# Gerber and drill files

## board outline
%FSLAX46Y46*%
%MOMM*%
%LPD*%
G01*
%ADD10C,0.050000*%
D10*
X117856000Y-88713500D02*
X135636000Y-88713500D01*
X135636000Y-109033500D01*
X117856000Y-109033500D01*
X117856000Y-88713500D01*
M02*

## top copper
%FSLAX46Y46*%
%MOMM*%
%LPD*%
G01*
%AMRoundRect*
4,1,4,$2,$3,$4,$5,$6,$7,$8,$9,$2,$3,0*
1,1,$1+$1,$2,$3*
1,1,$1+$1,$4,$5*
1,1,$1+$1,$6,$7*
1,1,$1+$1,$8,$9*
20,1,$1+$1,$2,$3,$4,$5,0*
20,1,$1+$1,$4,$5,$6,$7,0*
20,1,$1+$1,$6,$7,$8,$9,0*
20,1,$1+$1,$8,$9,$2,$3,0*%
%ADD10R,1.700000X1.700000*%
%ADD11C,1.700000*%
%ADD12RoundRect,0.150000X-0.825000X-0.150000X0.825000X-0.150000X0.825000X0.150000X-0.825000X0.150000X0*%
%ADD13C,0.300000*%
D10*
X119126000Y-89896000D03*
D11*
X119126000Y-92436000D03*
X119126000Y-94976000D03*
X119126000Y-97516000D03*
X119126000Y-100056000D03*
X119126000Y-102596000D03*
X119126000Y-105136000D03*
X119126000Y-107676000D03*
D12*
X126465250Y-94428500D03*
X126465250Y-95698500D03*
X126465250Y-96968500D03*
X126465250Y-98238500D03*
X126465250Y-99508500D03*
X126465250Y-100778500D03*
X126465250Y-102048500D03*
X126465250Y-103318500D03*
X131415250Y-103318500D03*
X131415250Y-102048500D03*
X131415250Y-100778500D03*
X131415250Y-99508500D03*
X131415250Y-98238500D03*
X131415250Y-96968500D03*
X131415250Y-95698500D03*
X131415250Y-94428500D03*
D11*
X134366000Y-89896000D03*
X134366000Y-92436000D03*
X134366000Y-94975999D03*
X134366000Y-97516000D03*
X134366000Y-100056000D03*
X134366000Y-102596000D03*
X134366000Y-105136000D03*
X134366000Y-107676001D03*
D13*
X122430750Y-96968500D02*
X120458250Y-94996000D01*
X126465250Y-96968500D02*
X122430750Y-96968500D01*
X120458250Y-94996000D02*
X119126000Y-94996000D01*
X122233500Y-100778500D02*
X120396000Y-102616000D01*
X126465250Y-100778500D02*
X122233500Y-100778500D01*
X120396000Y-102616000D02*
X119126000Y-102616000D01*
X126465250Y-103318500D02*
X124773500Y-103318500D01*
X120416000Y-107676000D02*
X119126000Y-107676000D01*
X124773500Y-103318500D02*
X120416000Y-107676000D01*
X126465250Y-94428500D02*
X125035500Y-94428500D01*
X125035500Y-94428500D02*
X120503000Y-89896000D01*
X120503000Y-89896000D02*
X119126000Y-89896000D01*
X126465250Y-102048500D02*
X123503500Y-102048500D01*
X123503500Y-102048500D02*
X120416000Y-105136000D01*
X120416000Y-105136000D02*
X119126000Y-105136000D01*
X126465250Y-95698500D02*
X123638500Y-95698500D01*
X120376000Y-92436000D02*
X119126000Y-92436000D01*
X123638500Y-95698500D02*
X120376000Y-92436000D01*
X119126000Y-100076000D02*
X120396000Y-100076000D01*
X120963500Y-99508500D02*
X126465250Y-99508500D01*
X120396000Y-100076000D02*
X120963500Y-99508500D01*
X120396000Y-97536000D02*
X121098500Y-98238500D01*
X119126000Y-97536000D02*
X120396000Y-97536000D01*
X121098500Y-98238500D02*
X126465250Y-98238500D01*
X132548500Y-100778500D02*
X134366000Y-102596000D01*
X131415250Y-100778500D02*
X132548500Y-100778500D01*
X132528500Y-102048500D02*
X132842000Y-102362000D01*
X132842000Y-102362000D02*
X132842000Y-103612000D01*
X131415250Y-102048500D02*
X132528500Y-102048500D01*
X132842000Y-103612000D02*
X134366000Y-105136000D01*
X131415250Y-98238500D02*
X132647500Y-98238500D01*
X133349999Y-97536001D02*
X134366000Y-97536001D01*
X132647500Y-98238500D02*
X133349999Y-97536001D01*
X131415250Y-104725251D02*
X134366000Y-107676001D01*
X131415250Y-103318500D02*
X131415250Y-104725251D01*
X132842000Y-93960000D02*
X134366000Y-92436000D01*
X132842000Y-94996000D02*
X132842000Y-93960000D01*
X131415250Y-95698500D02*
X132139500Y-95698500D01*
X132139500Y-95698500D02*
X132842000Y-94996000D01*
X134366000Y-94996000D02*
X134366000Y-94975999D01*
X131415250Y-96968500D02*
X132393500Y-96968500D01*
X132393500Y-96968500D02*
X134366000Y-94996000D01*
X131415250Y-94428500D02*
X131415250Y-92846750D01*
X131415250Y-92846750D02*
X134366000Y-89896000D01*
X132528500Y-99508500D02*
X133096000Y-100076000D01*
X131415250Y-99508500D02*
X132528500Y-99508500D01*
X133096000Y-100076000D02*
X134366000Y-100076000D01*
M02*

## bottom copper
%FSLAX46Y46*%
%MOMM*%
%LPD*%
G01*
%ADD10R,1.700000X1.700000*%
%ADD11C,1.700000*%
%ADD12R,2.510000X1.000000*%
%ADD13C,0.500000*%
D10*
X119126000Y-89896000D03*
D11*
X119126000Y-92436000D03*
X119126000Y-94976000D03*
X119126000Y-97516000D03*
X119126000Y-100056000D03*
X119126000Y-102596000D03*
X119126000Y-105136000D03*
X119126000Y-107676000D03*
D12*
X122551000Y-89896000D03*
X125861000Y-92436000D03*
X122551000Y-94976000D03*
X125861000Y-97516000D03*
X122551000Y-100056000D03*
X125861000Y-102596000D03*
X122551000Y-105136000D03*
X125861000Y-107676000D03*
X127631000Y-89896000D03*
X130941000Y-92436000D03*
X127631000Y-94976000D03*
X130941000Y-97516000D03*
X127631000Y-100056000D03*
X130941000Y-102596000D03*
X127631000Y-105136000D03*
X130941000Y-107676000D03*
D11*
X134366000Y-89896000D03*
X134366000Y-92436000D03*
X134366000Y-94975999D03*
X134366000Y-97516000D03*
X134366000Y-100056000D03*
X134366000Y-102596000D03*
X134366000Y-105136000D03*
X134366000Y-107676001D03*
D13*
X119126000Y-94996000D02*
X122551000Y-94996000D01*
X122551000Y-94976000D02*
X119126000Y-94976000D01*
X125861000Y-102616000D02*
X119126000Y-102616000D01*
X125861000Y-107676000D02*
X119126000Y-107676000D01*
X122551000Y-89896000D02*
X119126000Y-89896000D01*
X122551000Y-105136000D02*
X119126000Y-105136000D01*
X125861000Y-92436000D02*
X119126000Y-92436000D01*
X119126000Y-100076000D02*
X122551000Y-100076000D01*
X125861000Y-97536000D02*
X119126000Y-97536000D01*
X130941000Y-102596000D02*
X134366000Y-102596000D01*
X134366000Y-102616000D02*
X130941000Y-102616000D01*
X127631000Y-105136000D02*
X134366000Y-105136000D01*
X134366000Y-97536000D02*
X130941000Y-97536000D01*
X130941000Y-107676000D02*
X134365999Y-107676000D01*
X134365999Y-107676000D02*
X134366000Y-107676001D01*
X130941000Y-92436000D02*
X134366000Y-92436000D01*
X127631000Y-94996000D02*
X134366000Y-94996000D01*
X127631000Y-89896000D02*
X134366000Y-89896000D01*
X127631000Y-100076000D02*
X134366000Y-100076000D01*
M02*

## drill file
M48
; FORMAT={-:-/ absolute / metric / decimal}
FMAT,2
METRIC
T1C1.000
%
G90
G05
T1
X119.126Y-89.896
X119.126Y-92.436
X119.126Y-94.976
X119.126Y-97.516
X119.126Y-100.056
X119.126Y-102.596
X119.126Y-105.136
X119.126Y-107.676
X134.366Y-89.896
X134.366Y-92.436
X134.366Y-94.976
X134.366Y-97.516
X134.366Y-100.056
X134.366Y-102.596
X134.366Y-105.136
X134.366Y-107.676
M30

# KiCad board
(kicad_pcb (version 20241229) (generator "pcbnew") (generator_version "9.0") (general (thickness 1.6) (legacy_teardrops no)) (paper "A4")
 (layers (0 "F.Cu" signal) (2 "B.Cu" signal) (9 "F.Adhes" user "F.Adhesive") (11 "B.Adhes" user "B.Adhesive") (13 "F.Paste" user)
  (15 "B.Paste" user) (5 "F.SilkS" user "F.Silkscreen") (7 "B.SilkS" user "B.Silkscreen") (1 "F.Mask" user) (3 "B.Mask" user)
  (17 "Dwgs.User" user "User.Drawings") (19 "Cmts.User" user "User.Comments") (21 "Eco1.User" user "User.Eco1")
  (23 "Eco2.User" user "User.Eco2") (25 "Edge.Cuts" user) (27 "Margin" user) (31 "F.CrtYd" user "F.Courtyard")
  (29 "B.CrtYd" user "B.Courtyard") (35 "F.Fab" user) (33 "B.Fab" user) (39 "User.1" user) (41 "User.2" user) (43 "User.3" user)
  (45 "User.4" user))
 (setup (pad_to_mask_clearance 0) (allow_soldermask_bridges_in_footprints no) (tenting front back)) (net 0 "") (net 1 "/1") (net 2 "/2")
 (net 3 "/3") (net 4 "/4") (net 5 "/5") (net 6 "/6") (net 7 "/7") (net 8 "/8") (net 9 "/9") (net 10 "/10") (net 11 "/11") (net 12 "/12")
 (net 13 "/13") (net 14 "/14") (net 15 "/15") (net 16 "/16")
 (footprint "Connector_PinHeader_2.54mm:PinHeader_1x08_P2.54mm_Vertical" (layer "F.Cu") (at 119.126 89.896)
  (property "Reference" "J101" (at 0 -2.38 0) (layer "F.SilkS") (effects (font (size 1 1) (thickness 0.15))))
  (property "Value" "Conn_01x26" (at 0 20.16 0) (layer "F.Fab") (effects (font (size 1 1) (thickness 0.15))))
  (pad "1" thru_hole rect (at 0 0) (size 1.7 1.7) (drill 1) (layers "*.Cu" "*.Mask") (remove_unused_layers no) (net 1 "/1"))
  (pad "2" thru_hole circle (at 0 2.54) (size 1.7 1.7) (drill 1) (layers "*.Cu" "*.Mask") (remove_unused_layers no) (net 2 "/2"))
  (pad "3" thru_hole circle (at 0 5.08) (size 1.7 1.7) (drill 1) (layers "*.Cu" "*.Mask") (remove_unused_layers no) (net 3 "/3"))
  (pad "4" thru_hole circle (at 0 7.62) (size 1.7 1.7) (drill 1) (layers "*.Cu" "*.Mask") (remove_unused_layers no) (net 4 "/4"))
  (pad "5" thru_hole circle (at 0 10.16) (size 1.7 1.7) (drill 1) (layers "*.Cu" "*.Mask") (remove_unused_layers no) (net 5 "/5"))
  (pad "6" thru_hole circle (at 0 12.7) (size 1.7 1.7) (drill 1) (layers "*.Cu" "*.Mask") (remove_unused_layers no) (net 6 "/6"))
  (pad "7" thru_hole circle (at 0 15.24) (size 1.7 1.7) (drill 1) (layers "*.Cu" "*.Mask") (remove_unused_layers no) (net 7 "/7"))
  (pad "8" thru_hole circle (at 0 17.78) (size 1.7 1.7) (drill 1) (layers "*.Cu" "*.Mask") (remove_unused_layers no) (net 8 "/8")))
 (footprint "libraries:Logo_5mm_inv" (layer "F.Cu") (at 128.940483 91.168125)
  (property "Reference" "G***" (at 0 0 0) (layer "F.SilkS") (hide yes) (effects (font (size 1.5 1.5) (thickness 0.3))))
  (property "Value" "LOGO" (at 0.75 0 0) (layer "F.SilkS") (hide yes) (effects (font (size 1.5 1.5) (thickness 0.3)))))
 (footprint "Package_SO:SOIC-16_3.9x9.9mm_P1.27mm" (layer "F.Cu") (at 128.94025 98.8735)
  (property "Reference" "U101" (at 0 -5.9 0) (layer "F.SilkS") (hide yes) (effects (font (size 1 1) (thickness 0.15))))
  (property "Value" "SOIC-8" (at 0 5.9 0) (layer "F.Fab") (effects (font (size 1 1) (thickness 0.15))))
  (pad "1" smd roundrect (at -2.475 -4.445) (size 1.95 0.6) (layers "F.Cu" "F.Mask" "F.Paste") (roundrect_rratio 0.25) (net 1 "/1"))
  (pad "2" smd roundrect (at -2.475 -3.175) (size 1.95 0.6) (layers "F.Cu" "F.Mask" "F.Paste") (roundrect_rratio 0.25) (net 2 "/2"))
  (pad "3" smd roundrect (at -2.475 -1.905) (size 1.95 0.6) (layers "F.Cu" "F.Mask" "F.Paste") (roundrect_rratio 0.25) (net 3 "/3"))
  (pad "4" smd roundrect (at -2.475 -0.635) (size 1.95 0.6) (layers "F.Cu" "F.Mask" "F.Paste") (roundrect_rratio 0.25) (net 4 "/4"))
  (pad "5" smd roundrect (at -2.475 0.635) (size 1.95 0.6) (layers "F.Cu" "F.Mask" "F.Paste") (roundrect_rratio 0.25) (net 5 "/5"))
  (pad "6" smd roundrect (at -2.475 1.905) (size 1.95 0.6) (layers "F.Cu" "F.Mask" "F.Paste") (roundrect_rratio 0.25) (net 6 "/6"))
  (pad "7" smd roundrect (at -2.475 3.175) (size 1.95 0.6) (layers "F.Cu" "F.Mask" "F.Paste") (roundrect_rratio 0.25) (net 7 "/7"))
  (pad "8" smd roundrect (at -2.475 4.445) (size 1.95 0.6) (layers "F.Cu" "F.Mask" "F.Paste") (roundrect_rratio 0.25) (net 8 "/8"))
  (pad "9" smd roundrect (at 2.475 4.445) (size 1.95 0.6) (layers "F.Cu" "F.Mask" "F.Paste") (roundrect_rratio 0.25) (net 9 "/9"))
  (pad "10" smd roundrect (at 2.475 3.175) (size 1.95 0.6) (layers "F.Cu" "F.Mask" "F.Paste") (roundrect_rratio 0.25) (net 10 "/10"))
  (pad "11" smd roundrect (at 2.475 1.905) (size 1.95 0.6) (layers "F.Cu" "F.Mask" "F.Paste") (roundrect_rratio 0.25) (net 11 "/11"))
  (pad "12" smd roundrect (at 2.475 0.635) (size 1.95 0.6) (layers "F.Cu" "F.Mask" "F.Paste") (roundrect_rratio 0.25) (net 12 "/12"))
  (pad "13" smd roundrect (at 2.475 -0.635) (size 1.95 0.6) (layers "F.Cu" "F.Mask" "F.Paste") (roundrect_rratio 0.25) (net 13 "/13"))
  (pad "14" smd roundrect (at 2.475 -1.905) (size 1.95 0.6) (layers "F.Cu" "F.Mask" "F.Paste") (roundrect_rratio 0.25) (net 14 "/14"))
  (pad "15" smd roundrect (at 2.475 -3.175) (size 1.95 0.6) (layers "F.Cu" "F.Mask" "F.Paste") (roundrect_rratio 0.25) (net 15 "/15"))
  (pad "16" smd roundrect (at 2.475 -4.445) (size 1.95 0.6) (layers "F.Cu" "F.Mask" "F.Paste") (roundrect_rratio 0.25) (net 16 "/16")))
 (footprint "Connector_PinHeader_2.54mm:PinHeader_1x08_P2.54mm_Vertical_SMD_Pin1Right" (layer "B.Cu") (at 124.206 98.786 180)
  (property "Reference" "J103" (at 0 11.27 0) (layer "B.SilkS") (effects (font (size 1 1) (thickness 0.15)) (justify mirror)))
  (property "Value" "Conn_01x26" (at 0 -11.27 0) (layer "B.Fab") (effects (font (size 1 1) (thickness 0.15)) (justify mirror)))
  (pad "1" smd rect (at 1.655 8.89 180) (size 2.51 1) (layers "B.Cu" "B.Mask" "B.Paste") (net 1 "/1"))
  (pad "2" smd rect (at -1.655 6.35 180) (size 2.51 1) (layers "B.Cu" "B.Mask" "B.Paste") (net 2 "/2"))
  (pad "3" smd rect (at 1.655 3.81 180) (size 2.51 1) (layers "B.Cu" "B.Mask" "B.Paste") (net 3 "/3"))
  (pad "4" smd rect (at -1.655 1.27 180) (size 2.51 1) (layers "B.Cu" "B.Mask" "B.Paste") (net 4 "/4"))
  (pad "5" smd rect (at 1.655 -1.27 180) (size 2.51 1) (layers "B.Cu" "B.Mask" "B.Paste") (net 5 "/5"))
  (pad "6" smd rect (at -1.655 -3.81 180) (size 2.51 1) (layers "B.Cu" "B.Mask" "B.Paste") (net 6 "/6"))
  (pad "7" smd rect (at 1.655 -6.35 180) (size 2.51 1) (layers "B.Cu" "B.Mask" "B.Paste") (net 7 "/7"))
  (pad "8" smd rect (at -1.655 -8.89 180) (size 2.51 1) (layers "B.Cu" "B.Mask" "B.Paste") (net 8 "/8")))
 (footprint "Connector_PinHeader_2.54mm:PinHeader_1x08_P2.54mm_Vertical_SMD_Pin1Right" (layer "B.Cu") (at 129.286 98.786 180)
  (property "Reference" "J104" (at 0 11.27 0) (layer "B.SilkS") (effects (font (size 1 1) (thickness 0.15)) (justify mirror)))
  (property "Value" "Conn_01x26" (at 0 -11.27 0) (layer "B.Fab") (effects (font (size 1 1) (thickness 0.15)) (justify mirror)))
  (pad "1" smd rect (at 1.655 8.89 180) (size 2.51 1) (layers "B.Cu" "B.Mask" "B.Paste") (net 16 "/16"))
  (pad "2" smd rect (at -1.655 6.35 180) (size 2.51 1) (layers "B.Cu" "B.Mask" "B.Paste") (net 15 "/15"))
  (pad "3" smd rect (at 1.655 3.81 180) (size 2.51 1) (layers "B.Cu" "B.Mask" "B.Paste") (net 14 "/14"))
  (pad "4" smd rect (at -1.655 1.27 180) (size 2.51 1) (layers "B.Cu" "B.Mask" "B.Paste") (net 13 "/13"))
  (pad "5" smd rect (at 1.655 -1.27 180) (size 2.51 1) (layers "B.Cu" "B.Mask" "B.Paste") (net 12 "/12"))
  (pad "6" smd rect (at -1.655 -3.81 180) (size 2.51 1) (layers "B.Cu" "B.Mask" "B.Paste") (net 11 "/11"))
  (pad "7" smd rect (at 1.655 -6.35 180) (size 2.51 1) (layers "B.Cu" "B.Mask" "B.Paste") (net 10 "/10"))
  (pad "8" smd rect (at -1.655 -8.89 180) (size 2.51 1) (layers "B.Cu" "B.Mask" "B.Paste") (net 9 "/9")))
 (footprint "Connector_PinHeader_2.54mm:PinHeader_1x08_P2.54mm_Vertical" (layer "B.Cu") (at 134.366 89.896 180)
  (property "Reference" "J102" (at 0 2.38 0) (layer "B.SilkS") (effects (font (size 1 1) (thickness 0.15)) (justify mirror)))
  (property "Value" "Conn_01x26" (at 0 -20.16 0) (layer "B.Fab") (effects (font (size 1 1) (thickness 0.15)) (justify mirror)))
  (pad "1" thru_hole circle (at 0 0 180) (size 1.7 1.7) (drill 1) (layers "*.Cu" "*.Mask") (remove_unused_layers no) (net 16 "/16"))
  (pad "2" thru_hole circle (at 0 -2.54 180) (size 1.7 1.7) (drill 1) (layers "*.Cu" "*.Mask") (remove_unused_layers no) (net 15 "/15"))
  (pad "3" thru_hole circle (at 0 -5.079999 180) (size 1.7 1.7) (drill 1) (layers "*.Cu" "*.Mask") (remove_unused_layers no) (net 14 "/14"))
  (pad "4" thru_hole circle (at 0 -7.62 180) (size 1.7 1.7) (drill 1) (layers "*.Cu" "*.Mask") (remove_unused_layers no) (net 13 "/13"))
  (pad "5" thru_hole circle (at 0 -10.16 180) (size 1.7 1.7) (drill 1) (layers "*.Cu" "*.Mask") (remove_unused_layers no) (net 12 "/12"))
  (pad "6" thru_hole circle (at 0 -12.7 180) (size 1.7 1.7) (drill 1) (layers "*.Cu" "*.Mask") (remove_unused_layers no) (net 11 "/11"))
  (pad "7" thru_hole circle (at 0 -15.24 180) (size 1.7 1.7) (drill 1) (layers "*.Cu" "*.Mask") (remove_unused_layers no) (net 10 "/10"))
  (pad "8" thru_hole circle (at 0 -17.780001 180) (size 1.7 1.7) (drill 1) (layers "*.Cu" "*.Mask") (remove_unused_layers no) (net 9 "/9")))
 (gr_rect (start 117.856 88.7135) (end 135.636 109.0335) (stroke (width 0.05) (type default)) (fill no) (layer "Edge.Cuts"))
 (segment (start 122.43075 96.9685) (end 120.45825 94.996) (width 0.3) (layer "F.Cu") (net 3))
 (segment (start 126.46525 96.9685) (end 122.43075 96.9685) (width 0.3) (layer "F.Cu") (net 3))
 (segment (start 120.45825 94.996) (end 119.126 94.996) (width 0.3) (layer "F.Cu") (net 3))
 (segment (start 119.126 94.996) (end 122.551 94.996) (width 0.5) (layer "B.Cu") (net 3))
 (segment (start 122.551 94.976) (end 119.126 94.976) (width 0.5) (layer "B.Cu") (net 3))
 (segment (start 122.2335 100.7785) (end 120.396 102.616) (width 0.3) (layer "F.Cu") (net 6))
 (segment (start 126.46525 100.7785) (end 122.2335 100.7785) (width 0.3) (layer "F.Cu") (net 6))
 (segment (start 120.396 102.616) (end 119.126 102.616) (width 0.3) (layer "F.Cu") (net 6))
 (segment (start 125.861 102.616) (end 119.126 102.616) (width 0.5) (layer "B.Cu") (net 6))
 (segment (start 126.46525 103.3185) (end 124.7735 103.3185) (width 0.3) (layer "F.Cu") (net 8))
 (segment (start 120.416 107.676) (end 119.126 107.676) (width 0.3) (layer "F.Cu") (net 8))
 (segment (start 124.7735 103.3185) (end 120.416 107.676) (width 0.3) (layer "F.Cu") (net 8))
 (segment (start 125.861 107.676) (end 119.126 107.676) (width 0.5) (layer "B.Cu") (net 8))
 (segment (start 126.46525 94.4285) (end 125.0355 94.4285) (width 0.3) (layer "F.Cu") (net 1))
 (segment (start 125.0355 94.4285) (end 120.503 89.896) (width 0.3) (layer "F.Cu") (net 1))
 (segment (start 120.503 89.896) (end 119.126 89.896) (width 0.3) (layer "F.Cu") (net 1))
 (segment (start 122.551 89.896) (end 119.126 89.896) (width 0.5) (layer "B.Cu") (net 1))
 (segment (start 126.46525 102.0485) (end 123.5035 102.0485) (width 0.3) (layer "F.Cu") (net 7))
 (segment (start 123.5035 102.0485) (end 120.416 105.136) (width 0.3) (layer "F.Cu") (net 7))
 (segment (start 120.416 105.136) (end 119.126 105.136) (width 0.3) (layer "F.Cu") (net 7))
 (segment (start 122.551 105.136) (end 119.126 105.136) (width 0.5) (layer "B.Cu") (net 7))
 (segment (start 126.46525 95.6985) (end 123.6385 95.6985) (width 0.3) (layer "F.Cu") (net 2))
 (segment (start 120.376 92.436) (end 119.126 92.436) (width 0.3) (layer "F.Cu") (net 2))
 (segment (start 123.6385 95.6985) (end 120.376 92.436) (width 0.3) (layer "F.Cu") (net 2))
 (segment (start 125.861 92.436) (end 119.126 92.436) (width 0.5) (layer "B.Cu") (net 2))
 (segment (start 119.126 100.076) (end 120.396 100.076) (width 0.3) (layer "F.Cu") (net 5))
 (segment (start 120.9635 99.5085) (end 126.46525 99.5085) (width 0.3) (layer "F.Cu") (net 5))
 (segment (start 120.396 100.076) (end 120.9635 99.5085) (width 0.3) (layer "F.Cu") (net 5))
 (segment (start 119.126 100.076) (end 122.551 100.076) (width 0.5) (layer "B.Cu") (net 5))
 (segment (start 120.396 97.536) (end 121.0985 98.2385) (width 0.3) (layer "F.Cu") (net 4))
 (segment (start 119.126 97.536) (end 120.396 97.536) (width 0.3) (layer "F.Cu") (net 4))
 (segment (start 121.0985 98.2385) (end 126.46525 98.2385) (width 0.3) (layer "F.Cu") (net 4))
 (segment (start 125.861 97.536) (end 119.126 97.536) (width 0.5) (layer "B.Cu") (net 4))
 (segment (start 132.5485 100.7785) (end 134.366 102.596) (width 0.3) (layer "F.Cu") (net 11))
 (segment (start 131.41525 100.7785) (end 132.5485 100.7785) (width 0.3) (layer "F.Cu") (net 11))
 (segment (start 130.941 102.596) (end 134.366 102.596) (width 0.5) (layer "B.Cu") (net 11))
 (segment (start 134.366 102.616) (end 130.941 102.616) (width 0.5) (layer "B.Cu") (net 11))
 (segment (start 132.5285 102.0485) (end 132.842 102.362) (width 0.3) (layer "F.Cu") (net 10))
 (segment (start 132.842 102.362) (end 132.842 103.612) (width 0.3) (layer "F.Cu") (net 10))
 (segment (start 131.41525 102.0485) (end 132.5285 102.0485) (width 0.3) (layer "F.Cu") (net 10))
 (segment (start 132.842 103.612) (end 134.366 105.136) (width 0.3) (layer "F.Cu") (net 10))
 (segment (start 127.631 105.136) (end 134.366 105.136) (width 0.5) (layer "B.Cu") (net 10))
 (segment (start 131.41525 98.2385) (end 132.6475 98.2385) (width 0.3) (layer "F.Cu") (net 13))
 (segment (start 133.349999 97.536001) (end 134.366 97.536001) (width 0.3) (layer "F.Cu") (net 13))
 (segment (start 132.6475 98.2385) (end 133.349999 97.536001) (width 0.3) (layer "F.Cu") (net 13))
 (segment (start 134.366 97.536) (end 130.941 97.536) (width 0.5) (layer "B.Cu") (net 13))
 (segment (start 131.41525 104.725251) (end 134.366 107.676001) (width 0.3) (layer "F.Cu") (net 9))
 (segment (start 131.41525 103.3185) (end 131.41525 104.725251) (width 0.3) (layer "F.Cu") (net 9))
 (segment (start 130.941 107.676) (end 134.365999 107.676) (width 0.5) (layer "B.Cu") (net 9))
 (segment (start 134.365999 107.676) (end 134.366 107.676001) (width 0.5) (layer "B.Cu") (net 9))
 (segment (start 132.842 93.96) (end 134.366 92.436) (width 0.3) (layer "F.Cu") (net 15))
 (segment (start 132.842 94.996) (end 132.842 93.96) (width 0.3) (layer "F.Cu") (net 15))
 (segment (start 131.41525 95.6985) (end 132.1395 95.6985) (width 0.3) (layer "F.Cu") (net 15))
 (segment (start 132.1395 95.6985) (end 132.842 94.996) (width 0.3) (layer "F.Cu") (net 15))
 (segment (start 130.941 92.436) (end 134.366 92.436) (width 0.5) (layer "B.Cu") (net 15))
 (segment (start 134.366 94.996) (end 134.366 94.975999) (width 0.3) (layer "F.Cu") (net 14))
 (segment (start 131.41525 96.9685) (end 132.3935 96.9685) (width 0.3) (layer "F.Cu") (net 14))
 (segment (start 132.3935 96.9685) (end 134.366 94.996) (width 0.3) (layer "F.Cu") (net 14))
 (segment (start 127.631 94.996) (end 134.366 94.996) (width 0.5) (layer "B.Cu") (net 14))
 (segment (start 131.41525 94.4285) (end 131.41525 92.84675) (width 0.3) (layer "F.Cu") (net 16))
 (segment (start 131.41525 92.84675) (end 134.366 89.896) (width 0.3) (layer "F.Cu") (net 16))
 (segment (start 127.631 89.896) (end 134.366 89.896) (width 0.5) (layer "B.Cu") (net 16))
 (segment (start 132.5285 99.5085) (end 133.096 100.076) (width 0.3) (layer "F.Cu") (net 12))
 (segment (start 131.41525 99.5085) (end 132.5285 99.5085) (width 0.3) (layer "F.Cu") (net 12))
 (segment (start 133.096 100.076) (end 134.366 100.076) (width 0.3) (layer "F.Cu") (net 12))
 (segment (start 127.631 100.076) (end 134.366 100.076) (width 0.5) (layer "B.Cu") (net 12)))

